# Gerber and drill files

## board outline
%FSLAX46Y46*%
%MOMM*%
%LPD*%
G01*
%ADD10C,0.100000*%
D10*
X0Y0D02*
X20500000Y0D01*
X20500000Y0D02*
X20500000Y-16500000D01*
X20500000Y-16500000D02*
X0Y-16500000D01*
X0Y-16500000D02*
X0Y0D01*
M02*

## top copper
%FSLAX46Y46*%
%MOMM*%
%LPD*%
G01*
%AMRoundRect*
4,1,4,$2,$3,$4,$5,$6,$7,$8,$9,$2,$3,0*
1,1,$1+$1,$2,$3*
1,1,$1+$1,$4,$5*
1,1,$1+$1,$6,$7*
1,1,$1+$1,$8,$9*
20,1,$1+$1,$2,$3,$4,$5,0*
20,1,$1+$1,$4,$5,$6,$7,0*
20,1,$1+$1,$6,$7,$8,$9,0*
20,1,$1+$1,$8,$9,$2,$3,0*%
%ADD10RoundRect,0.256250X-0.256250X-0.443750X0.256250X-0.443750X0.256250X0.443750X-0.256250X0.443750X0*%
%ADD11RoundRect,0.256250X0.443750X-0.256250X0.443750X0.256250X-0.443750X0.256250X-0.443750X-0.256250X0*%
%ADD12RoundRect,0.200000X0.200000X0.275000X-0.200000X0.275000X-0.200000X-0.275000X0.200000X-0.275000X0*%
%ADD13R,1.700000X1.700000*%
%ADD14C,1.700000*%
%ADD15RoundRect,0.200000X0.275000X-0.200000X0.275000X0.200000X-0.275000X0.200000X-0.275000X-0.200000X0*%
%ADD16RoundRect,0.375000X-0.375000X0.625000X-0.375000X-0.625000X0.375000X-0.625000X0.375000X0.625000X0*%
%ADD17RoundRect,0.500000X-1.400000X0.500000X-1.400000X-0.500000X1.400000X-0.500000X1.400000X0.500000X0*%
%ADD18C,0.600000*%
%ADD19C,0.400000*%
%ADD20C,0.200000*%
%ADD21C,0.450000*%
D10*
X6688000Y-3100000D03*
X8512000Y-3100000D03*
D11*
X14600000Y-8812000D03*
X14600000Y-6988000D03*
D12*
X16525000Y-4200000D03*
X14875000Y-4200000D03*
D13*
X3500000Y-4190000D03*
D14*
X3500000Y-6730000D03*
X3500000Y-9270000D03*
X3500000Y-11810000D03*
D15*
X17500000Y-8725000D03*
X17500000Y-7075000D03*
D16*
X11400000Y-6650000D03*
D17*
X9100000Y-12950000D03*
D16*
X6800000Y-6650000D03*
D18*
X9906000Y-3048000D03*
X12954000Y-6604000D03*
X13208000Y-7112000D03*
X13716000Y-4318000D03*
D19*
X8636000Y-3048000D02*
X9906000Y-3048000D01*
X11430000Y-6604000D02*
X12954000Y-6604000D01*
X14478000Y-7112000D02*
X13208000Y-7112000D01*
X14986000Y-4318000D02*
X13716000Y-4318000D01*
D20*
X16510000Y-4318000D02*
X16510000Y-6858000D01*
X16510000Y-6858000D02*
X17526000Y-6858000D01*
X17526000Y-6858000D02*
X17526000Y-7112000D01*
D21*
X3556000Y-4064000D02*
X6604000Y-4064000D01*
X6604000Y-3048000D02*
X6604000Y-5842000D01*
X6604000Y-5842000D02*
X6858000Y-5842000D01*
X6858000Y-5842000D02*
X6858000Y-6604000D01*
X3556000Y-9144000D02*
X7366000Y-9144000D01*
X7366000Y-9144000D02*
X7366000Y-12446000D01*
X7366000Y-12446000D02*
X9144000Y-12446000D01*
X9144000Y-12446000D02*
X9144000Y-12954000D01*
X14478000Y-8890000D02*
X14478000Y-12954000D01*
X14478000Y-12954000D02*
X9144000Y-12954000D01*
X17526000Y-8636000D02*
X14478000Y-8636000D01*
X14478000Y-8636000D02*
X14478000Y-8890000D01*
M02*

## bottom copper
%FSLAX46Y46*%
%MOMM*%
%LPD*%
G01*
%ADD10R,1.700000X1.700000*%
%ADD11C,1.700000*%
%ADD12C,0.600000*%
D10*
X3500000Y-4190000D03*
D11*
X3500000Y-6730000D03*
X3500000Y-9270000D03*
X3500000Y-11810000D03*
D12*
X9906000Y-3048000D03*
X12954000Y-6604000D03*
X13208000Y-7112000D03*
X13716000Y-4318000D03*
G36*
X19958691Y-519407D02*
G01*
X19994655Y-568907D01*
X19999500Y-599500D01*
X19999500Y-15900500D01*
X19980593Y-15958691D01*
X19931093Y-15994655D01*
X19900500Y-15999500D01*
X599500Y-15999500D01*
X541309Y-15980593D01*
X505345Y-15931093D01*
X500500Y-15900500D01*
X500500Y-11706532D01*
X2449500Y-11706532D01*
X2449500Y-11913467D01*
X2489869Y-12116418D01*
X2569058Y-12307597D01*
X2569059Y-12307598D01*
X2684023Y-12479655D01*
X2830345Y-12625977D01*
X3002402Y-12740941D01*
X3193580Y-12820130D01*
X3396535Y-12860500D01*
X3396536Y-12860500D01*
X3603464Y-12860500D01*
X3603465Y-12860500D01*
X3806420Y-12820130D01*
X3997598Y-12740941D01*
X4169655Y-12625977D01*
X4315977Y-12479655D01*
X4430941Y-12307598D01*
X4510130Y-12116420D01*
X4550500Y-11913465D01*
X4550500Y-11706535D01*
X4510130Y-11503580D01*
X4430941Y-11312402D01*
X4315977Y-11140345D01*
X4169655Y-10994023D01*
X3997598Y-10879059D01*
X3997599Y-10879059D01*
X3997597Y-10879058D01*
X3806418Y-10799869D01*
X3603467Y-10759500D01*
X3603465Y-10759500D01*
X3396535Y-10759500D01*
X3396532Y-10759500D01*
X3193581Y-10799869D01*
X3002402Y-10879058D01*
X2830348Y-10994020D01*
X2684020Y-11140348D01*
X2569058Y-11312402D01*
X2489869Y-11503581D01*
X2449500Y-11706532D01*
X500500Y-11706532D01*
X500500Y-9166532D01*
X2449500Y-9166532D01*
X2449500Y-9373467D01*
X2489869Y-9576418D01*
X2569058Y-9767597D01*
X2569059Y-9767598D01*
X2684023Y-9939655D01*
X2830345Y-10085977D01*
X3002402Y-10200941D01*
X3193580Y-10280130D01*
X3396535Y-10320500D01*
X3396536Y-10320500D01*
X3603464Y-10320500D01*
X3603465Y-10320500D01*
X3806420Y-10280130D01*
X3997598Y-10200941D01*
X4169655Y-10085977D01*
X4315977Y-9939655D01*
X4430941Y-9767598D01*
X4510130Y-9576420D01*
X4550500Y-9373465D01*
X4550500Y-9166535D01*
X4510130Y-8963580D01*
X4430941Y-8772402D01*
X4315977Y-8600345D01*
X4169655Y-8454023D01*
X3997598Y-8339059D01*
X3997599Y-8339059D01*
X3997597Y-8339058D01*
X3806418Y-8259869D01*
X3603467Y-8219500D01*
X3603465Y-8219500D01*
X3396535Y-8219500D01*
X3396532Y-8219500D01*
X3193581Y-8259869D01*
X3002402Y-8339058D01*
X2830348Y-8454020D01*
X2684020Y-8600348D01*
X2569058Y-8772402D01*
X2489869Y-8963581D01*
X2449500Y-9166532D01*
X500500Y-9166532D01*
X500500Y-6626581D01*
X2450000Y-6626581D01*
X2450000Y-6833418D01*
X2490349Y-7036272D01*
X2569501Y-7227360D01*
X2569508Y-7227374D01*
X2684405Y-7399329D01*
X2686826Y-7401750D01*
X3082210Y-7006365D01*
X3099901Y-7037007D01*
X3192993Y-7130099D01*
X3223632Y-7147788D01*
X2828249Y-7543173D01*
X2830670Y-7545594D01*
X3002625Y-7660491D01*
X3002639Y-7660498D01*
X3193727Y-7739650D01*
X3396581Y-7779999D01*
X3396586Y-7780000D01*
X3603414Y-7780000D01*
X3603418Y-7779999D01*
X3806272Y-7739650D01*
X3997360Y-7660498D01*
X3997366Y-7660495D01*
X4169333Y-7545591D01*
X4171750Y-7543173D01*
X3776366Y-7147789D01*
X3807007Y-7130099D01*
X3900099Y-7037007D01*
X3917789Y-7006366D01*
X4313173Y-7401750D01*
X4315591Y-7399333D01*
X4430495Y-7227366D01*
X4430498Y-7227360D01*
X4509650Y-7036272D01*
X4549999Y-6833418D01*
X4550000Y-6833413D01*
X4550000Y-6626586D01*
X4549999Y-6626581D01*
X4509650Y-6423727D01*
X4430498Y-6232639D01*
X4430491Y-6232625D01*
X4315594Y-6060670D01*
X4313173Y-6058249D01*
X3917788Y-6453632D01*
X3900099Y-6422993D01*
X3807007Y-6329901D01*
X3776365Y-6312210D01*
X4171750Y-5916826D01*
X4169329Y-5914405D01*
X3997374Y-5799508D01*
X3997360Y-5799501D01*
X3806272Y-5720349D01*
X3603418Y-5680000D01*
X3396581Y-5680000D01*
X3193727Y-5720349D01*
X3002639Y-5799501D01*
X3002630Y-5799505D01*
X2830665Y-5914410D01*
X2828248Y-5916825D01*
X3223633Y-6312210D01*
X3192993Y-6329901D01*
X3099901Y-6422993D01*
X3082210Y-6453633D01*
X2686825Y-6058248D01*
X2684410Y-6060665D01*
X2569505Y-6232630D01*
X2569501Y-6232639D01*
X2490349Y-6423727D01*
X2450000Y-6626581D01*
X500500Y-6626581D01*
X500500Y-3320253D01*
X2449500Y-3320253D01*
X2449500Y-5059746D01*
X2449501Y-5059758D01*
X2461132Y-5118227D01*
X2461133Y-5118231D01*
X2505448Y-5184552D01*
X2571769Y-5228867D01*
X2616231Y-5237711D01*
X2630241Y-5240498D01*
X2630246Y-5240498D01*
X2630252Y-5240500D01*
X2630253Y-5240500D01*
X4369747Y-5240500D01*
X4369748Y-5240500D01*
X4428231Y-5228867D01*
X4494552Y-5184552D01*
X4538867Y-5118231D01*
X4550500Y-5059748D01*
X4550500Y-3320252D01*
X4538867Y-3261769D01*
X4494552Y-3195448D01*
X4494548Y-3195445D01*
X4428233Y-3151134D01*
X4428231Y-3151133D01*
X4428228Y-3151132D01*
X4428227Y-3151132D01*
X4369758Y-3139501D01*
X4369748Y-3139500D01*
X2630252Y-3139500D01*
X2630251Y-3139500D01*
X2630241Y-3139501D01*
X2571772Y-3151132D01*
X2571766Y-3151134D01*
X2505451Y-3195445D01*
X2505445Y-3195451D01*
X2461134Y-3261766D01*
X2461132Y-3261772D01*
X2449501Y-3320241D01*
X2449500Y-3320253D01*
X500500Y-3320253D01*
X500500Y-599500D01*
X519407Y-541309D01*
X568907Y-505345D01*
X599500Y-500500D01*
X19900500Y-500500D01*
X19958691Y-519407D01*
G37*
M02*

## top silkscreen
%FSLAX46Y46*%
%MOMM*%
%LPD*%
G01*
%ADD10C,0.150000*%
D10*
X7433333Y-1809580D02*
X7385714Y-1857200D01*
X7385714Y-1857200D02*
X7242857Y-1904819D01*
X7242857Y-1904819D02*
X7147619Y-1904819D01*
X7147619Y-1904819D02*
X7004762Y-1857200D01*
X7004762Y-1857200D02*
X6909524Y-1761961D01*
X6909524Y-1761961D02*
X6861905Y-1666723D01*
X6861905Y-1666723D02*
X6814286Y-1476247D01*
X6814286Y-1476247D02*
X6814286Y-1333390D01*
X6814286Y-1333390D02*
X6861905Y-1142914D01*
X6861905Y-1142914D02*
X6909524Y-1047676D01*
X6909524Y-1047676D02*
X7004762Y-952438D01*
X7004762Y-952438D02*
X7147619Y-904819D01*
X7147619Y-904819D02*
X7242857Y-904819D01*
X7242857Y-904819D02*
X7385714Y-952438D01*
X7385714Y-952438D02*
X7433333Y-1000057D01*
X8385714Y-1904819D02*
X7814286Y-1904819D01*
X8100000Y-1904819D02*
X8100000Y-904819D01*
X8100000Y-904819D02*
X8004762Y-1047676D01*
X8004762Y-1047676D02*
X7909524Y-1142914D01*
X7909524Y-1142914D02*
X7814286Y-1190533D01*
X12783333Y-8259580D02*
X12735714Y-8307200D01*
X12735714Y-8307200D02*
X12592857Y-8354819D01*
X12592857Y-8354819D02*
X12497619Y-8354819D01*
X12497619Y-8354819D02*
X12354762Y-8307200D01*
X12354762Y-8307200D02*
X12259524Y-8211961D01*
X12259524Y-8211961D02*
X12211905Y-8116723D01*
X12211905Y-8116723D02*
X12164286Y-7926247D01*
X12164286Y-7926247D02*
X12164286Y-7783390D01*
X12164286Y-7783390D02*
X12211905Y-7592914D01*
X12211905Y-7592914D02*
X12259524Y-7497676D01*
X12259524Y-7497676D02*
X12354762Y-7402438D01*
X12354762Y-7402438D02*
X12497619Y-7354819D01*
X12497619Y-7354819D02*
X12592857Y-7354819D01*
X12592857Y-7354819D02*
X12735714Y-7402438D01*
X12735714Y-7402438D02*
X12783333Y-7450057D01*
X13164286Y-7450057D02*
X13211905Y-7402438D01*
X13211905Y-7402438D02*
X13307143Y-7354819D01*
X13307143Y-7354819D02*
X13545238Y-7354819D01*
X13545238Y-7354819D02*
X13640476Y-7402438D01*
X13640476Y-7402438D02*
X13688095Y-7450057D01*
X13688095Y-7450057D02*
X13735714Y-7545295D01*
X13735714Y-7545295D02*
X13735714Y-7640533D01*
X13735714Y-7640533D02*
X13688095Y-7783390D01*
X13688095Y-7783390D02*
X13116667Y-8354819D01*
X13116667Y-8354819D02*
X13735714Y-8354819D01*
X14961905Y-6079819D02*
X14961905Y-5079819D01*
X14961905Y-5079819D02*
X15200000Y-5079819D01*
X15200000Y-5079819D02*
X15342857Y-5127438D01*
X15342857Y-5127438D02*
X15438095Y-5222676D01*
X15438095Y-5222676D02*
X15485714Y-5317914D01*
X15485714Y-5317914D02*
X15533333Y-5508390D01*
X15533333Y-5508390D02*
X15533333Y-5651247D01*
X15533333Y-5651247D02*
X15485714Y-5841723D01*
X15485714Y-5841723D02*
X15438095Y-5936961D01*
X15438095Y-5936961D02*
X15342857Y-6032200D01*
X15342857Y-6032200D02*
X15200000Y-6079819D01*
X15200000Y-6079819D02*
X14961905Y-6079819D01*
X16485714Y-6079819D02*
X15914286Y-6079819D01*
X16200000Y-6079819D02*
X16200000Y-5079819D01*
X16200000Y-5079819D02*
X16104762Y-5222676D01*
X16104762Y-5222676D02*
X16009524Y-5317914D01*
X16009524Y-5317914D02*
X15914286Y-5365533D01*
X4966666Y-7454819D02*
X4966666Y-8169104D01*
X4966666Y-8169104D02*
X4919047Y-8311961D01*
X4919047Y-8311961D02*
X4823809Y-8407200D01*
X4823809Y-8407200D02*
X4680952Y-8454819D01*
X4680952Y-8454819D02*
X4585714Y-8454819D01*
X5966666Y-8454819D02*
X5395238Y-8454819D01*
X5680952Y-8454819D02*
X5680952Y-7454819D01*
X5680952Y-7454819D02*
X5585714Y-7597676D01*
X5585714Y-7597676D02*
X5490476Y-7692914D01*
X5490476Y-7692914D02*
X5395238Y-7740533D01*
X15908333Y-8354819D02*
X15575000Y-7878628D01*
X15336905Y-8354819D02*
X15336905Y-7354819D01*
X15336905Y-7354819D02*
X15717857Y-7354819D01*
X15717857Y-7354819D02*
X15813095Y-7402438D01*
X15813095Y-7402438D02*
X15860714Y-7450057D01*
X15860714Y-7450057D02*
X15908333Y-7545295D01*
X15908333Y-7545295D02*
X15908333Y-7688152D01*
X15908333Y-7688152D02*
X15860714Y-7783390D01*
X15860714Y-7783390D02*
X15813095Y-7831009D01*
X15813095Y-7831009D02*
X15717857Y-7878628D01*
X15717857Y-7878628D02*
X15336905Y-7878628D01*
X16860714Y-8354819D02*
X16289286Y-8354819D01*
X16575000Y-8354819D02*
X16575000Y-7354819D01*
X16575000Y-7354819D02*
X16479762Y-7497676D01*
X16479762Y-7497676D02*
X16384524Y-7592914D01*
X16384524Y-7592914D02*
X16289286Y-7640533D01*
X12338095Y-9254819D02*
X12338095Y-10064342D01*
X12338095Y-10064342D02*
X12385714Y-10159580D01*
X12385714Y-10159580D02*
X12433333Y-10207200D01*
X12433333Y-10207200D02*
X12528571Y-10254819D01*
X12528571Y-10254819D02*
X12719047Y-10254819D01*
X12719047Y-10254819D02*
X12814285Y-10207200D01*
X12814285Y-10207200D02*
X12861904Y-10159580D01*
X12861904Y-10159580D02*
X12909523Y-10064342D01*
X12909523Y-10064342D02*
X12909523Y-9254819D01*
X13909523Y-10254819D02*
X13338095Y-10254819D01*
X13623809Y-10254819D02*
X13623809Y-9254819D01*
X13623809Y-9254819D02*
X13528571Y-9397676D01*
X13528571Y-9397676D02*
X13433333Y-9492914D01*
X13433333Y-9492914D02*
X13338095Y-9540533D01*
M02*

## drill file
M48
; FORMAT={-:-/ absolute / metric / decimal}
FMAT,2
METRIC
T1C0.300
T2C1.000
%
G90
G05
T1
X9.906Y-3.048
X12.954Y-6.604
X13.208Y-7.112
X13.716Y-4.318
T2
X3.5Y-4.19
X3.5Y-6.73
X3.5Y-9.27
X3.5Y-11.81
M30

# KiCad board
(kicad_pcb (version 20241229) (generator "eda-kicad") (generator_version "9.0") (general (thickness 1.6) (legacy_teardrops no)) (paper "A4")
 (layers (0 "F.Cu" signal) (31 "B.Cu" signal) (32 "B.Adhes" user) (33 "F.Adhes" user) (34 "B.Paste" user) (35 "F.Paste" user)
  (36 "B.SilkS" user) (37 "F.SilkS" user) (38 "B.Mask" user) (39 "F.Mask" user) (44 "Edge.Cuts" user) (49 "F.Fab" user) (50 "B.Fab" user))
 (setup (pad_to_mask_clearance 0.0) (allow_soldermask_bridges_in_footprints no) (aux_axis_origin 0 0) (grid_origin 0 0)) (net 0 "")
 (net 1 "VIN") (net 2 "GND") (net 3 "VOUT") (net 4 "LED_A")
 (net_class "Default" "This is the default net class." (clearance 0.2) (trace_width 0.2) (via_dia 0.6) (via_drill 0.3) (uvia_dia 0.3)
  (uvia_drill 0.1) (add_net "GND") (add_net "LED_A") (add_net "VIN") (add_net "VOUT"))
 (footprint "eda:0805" (layer "F.Cu") (at 7.6 3.1 0)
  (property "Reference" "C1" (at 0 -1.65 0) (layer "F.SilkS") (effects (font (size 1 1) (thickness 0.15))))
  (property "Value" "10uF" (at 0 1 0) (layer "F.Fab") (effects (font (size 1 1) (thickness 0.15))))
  (pad "1" smd roundrect (at -0.912 0 0) (size 1.025 1.4) (roundrect_rratio 0.25) (layers "F.Cu" "F.Paste" "F.Mask") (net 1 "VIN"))
  (pad "2" smd roundrect (at 0.912 0 0) (size 1.025 1.4) (roundrect_rratio 0.25) (layers "F.Cu" "F.Paste" "F.Mask") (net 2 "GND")))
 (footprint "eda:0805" (layer "F.Cu") (at 14.6 7.9 -270)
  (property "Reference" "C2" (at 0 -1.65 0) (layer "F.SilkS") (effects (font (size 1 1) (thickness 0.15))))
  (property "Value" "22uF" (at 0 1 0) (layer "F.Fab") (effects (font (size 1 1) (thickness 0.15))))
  (pad "1" smd roundrect (at -0.912 0 -270) (size 1.025 1.4) (roundrect_rratio 0.25) (layers "F.Cu" "F.Paste" "F.Mask") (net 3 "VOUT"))
  (pad "2" smd roundrect (at 0.912 0 -270) (size 1.025 1.4) (roundrect_rratio 0.25) (layers "F.Cu" "F.Paste" "F.Mask") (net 2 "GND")))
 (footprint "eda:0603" (layer "F.Cu") (at 15.7 4.2 -180)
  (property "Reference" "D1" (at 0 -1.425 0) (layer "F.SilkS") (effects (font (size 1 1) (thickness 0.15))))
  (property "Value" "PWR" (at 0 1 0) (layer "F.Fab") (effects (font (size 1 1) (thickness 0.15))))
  (pad "1" smd roundrect (at -0.825 0 -180) (size 0.8 0.95) (roundrect_rratio 0.25) (layers "F.Cu" "F.Paste" "F.Mask") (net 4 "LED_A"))
  (pad "2" smd roundrect (at 0.825 0 -180) (size 0.8 0.95) (roundrect_rratio 0.25) (layers "F.Cu" "F.Paste" "F.Mask") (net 2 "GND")))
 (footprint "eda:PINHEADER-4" (layer "F.Cu") (at 3.5 8 -90)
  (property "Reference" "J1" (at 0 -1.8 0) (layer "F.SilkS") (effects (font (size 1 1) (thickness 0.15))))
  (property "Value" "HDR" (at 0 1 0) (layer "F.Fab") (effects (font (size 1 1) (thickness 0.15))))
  (pad "1" thru_hole rect (at -3.81 0 -90) (size 1.7 1.7) (drill 1) (layers "*.Cu" "*.Mask") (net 1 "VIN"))
  (pad "2" thru_hole circle (at -1.27 0 -90) (size 1.7 1.7) (drill 1) (layers "*.Cu" "*.Mask") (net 2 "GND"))
  (pad "3" thru_hole circle (at 1.27 0 -90) (size 1.7 1.7) (drill 1) (layers "*.Cu" "*.Mask") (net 3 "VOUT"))
  (pad "4" thru_hole circle (at 3.81 0 -90) (size 1.7 1.7) (drill 1) (layers "*.Cu" "*.Mask")))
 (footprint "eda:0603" (layer "F.Cu") (at 17.5 7.9 -270)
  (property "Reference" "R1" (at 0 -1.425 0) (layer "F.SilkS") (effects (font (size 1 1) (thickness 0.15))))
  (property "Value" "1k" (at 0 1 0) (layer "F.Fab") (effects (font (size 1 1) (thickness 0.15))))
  (pad "1" smd roundrect (at -0.825 0 -270) (size 0.8 0.95) (roundrect_rratio 0.25) (layers "F.Cu" "F.Paste" "F.Mask") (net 3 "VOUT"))
  (pad "2" smd roundrect (at 0.825 0 -270) (size 0.8 0.95) (roundrect_rratio 0.25) (layers "F.Cu" "F.Paste" "F.Mask") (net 4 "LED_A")))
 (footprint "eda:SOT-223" (layer "F.Cu") (at 9.1 9.8 -90)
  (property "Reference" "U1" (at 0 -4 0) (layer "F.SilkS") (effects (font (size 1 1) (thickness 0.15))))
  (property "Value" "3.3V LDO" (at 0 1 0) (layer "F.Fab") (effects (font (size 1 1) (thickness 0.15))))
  (pad "1" smd roundrect (at -3.15 -2.3 -90) (size 2 1.5) (roundrect_rratio 0.25) (layers "F.Cu" "F.Paste" "F.Mask") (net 2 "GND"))
  (pad "2" smd roundrect (at 3.15 0 -90) (size 2 3.8) (roundrect_rratio 0.25) (layers "F.Cu" "F.Paste" "F.Mask") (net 3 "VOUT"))
  (pad "3" smd roundrect (at -3.15 2.3 -90) (size 2 1.5) (roundrect_rratio 0.25) (layers "F.Cu" "F.Paste" "F.Mask") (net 1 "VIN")))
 (segment (start 8.636 3.048) (end 9.906 3.048) (width 0.4) (layer "F.Cu") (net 2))
 (segment (start 11.43 6.604) (end 12.954 6.604) (width 0.4) (layer "F.Cu") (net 2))
 (segment (start 14.478 7.112) (end 13.208 7.112) (width 0.4) (layer "F.Cu") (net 2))
 (segment (start 14.986 4.318) (end 13.716 4.318) (width 0.4) (layer "F.Cu") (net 2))
 (segment (start 16.51 4.318) (end 16.51 6.858) (width 0.2) (layer "F.Cu") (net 4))
 (segment (start 16.51 6.858) (end 17.526 6.858) (width 0.2) (layer "F.Cu") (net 4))
 (segment (start 17.526 6.858) (end 17.526 7.112) (width 0.2) (layer "F.Cu") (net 4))
 (segment (start 3.556 4.064) (end 6.604 4.064) (width 0.45) (layer "F.Cu") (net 1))
 (segment (start 6.604 3.048) (end 6.604 5.842) (width 0.45) (layer "F.Cu") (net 1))
 (segment (start 6.604 5.842) (end 6.858 5.842) (width 0.45) (layer "F.Cu") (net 1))
 (segment (start 6.858 5.842) (end 6.858 6.604) (width 0.45) (layer "F.Cu") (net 1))
 (segment (start 3.556 9.144) (end 7.366 9.144) (width 0.45) (layer "F.Cu") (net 3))
 (segment (start 7.366 9.144) (end 7.366 12.446) (width 0.45) (layer "F.Cu") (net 3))
 (segment (start 7.366 12.446) (end 9.144 12.446) (width 0.45) (layer "F.Cu") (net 3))
 (segment (start 9.144 12.446) (end 9.144 12.954) (width 0.45) (layer "F.Cu") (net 3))
 (segment (start 14.478 8.89) (end 14.478 12.954) (width 0.45) (layer "F.Cu") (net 3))
 (segment (start 14.478 12.954) (end 9.144 12.954) (width 0.45) (layer "F.Cu") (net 3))
 (segment (start 17.526 8.636) (end 14.478 8.636) (width 0.45) (layer "F.Cu") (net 3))
 (segment (start 14.478 8.636) (end 14.478 8.89) (width 0.45) (layer "F.Cu") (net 3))
 (via (at 9.906 3.048) (size 0.6) (drill 0.3) (layers "F.Cu" "B.Cu") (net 2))
 (via (at 12.954 6.604) (size 0.6) (drill 0.3) (layers "F.Cu" "B.Cu") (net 2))
 (via (at 13.208 7.112) (size 0.6) (drill 0.3) (layers "F.Cu" "B.Cu") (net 2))
 (via (at 13.716 4.318) (size 0.6) (drill 0.3) (layers "F.Cu" "B.Cu") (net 2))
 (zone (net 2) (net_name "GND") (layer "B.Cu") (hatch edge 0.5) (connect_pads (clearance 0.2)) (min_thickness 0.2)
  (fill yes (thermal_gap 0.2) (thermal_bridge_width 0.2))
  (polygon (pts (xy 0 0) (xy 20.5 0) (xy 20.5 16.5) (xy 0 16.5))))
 (gr_line (start 0 0) (end 20.5 0) (layer "Edge.Cuts")) (gr_line (start 20.5 0) (end 20.5 16.5) (layer "Edge.Cuts"))
 (gr_line (start 20.5 16.5) (end 0 16.5) (layer "Edge.Cuts")) (gr_line (start 0 16.5) (end 0 0) (layer "Edge.Cuts")))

